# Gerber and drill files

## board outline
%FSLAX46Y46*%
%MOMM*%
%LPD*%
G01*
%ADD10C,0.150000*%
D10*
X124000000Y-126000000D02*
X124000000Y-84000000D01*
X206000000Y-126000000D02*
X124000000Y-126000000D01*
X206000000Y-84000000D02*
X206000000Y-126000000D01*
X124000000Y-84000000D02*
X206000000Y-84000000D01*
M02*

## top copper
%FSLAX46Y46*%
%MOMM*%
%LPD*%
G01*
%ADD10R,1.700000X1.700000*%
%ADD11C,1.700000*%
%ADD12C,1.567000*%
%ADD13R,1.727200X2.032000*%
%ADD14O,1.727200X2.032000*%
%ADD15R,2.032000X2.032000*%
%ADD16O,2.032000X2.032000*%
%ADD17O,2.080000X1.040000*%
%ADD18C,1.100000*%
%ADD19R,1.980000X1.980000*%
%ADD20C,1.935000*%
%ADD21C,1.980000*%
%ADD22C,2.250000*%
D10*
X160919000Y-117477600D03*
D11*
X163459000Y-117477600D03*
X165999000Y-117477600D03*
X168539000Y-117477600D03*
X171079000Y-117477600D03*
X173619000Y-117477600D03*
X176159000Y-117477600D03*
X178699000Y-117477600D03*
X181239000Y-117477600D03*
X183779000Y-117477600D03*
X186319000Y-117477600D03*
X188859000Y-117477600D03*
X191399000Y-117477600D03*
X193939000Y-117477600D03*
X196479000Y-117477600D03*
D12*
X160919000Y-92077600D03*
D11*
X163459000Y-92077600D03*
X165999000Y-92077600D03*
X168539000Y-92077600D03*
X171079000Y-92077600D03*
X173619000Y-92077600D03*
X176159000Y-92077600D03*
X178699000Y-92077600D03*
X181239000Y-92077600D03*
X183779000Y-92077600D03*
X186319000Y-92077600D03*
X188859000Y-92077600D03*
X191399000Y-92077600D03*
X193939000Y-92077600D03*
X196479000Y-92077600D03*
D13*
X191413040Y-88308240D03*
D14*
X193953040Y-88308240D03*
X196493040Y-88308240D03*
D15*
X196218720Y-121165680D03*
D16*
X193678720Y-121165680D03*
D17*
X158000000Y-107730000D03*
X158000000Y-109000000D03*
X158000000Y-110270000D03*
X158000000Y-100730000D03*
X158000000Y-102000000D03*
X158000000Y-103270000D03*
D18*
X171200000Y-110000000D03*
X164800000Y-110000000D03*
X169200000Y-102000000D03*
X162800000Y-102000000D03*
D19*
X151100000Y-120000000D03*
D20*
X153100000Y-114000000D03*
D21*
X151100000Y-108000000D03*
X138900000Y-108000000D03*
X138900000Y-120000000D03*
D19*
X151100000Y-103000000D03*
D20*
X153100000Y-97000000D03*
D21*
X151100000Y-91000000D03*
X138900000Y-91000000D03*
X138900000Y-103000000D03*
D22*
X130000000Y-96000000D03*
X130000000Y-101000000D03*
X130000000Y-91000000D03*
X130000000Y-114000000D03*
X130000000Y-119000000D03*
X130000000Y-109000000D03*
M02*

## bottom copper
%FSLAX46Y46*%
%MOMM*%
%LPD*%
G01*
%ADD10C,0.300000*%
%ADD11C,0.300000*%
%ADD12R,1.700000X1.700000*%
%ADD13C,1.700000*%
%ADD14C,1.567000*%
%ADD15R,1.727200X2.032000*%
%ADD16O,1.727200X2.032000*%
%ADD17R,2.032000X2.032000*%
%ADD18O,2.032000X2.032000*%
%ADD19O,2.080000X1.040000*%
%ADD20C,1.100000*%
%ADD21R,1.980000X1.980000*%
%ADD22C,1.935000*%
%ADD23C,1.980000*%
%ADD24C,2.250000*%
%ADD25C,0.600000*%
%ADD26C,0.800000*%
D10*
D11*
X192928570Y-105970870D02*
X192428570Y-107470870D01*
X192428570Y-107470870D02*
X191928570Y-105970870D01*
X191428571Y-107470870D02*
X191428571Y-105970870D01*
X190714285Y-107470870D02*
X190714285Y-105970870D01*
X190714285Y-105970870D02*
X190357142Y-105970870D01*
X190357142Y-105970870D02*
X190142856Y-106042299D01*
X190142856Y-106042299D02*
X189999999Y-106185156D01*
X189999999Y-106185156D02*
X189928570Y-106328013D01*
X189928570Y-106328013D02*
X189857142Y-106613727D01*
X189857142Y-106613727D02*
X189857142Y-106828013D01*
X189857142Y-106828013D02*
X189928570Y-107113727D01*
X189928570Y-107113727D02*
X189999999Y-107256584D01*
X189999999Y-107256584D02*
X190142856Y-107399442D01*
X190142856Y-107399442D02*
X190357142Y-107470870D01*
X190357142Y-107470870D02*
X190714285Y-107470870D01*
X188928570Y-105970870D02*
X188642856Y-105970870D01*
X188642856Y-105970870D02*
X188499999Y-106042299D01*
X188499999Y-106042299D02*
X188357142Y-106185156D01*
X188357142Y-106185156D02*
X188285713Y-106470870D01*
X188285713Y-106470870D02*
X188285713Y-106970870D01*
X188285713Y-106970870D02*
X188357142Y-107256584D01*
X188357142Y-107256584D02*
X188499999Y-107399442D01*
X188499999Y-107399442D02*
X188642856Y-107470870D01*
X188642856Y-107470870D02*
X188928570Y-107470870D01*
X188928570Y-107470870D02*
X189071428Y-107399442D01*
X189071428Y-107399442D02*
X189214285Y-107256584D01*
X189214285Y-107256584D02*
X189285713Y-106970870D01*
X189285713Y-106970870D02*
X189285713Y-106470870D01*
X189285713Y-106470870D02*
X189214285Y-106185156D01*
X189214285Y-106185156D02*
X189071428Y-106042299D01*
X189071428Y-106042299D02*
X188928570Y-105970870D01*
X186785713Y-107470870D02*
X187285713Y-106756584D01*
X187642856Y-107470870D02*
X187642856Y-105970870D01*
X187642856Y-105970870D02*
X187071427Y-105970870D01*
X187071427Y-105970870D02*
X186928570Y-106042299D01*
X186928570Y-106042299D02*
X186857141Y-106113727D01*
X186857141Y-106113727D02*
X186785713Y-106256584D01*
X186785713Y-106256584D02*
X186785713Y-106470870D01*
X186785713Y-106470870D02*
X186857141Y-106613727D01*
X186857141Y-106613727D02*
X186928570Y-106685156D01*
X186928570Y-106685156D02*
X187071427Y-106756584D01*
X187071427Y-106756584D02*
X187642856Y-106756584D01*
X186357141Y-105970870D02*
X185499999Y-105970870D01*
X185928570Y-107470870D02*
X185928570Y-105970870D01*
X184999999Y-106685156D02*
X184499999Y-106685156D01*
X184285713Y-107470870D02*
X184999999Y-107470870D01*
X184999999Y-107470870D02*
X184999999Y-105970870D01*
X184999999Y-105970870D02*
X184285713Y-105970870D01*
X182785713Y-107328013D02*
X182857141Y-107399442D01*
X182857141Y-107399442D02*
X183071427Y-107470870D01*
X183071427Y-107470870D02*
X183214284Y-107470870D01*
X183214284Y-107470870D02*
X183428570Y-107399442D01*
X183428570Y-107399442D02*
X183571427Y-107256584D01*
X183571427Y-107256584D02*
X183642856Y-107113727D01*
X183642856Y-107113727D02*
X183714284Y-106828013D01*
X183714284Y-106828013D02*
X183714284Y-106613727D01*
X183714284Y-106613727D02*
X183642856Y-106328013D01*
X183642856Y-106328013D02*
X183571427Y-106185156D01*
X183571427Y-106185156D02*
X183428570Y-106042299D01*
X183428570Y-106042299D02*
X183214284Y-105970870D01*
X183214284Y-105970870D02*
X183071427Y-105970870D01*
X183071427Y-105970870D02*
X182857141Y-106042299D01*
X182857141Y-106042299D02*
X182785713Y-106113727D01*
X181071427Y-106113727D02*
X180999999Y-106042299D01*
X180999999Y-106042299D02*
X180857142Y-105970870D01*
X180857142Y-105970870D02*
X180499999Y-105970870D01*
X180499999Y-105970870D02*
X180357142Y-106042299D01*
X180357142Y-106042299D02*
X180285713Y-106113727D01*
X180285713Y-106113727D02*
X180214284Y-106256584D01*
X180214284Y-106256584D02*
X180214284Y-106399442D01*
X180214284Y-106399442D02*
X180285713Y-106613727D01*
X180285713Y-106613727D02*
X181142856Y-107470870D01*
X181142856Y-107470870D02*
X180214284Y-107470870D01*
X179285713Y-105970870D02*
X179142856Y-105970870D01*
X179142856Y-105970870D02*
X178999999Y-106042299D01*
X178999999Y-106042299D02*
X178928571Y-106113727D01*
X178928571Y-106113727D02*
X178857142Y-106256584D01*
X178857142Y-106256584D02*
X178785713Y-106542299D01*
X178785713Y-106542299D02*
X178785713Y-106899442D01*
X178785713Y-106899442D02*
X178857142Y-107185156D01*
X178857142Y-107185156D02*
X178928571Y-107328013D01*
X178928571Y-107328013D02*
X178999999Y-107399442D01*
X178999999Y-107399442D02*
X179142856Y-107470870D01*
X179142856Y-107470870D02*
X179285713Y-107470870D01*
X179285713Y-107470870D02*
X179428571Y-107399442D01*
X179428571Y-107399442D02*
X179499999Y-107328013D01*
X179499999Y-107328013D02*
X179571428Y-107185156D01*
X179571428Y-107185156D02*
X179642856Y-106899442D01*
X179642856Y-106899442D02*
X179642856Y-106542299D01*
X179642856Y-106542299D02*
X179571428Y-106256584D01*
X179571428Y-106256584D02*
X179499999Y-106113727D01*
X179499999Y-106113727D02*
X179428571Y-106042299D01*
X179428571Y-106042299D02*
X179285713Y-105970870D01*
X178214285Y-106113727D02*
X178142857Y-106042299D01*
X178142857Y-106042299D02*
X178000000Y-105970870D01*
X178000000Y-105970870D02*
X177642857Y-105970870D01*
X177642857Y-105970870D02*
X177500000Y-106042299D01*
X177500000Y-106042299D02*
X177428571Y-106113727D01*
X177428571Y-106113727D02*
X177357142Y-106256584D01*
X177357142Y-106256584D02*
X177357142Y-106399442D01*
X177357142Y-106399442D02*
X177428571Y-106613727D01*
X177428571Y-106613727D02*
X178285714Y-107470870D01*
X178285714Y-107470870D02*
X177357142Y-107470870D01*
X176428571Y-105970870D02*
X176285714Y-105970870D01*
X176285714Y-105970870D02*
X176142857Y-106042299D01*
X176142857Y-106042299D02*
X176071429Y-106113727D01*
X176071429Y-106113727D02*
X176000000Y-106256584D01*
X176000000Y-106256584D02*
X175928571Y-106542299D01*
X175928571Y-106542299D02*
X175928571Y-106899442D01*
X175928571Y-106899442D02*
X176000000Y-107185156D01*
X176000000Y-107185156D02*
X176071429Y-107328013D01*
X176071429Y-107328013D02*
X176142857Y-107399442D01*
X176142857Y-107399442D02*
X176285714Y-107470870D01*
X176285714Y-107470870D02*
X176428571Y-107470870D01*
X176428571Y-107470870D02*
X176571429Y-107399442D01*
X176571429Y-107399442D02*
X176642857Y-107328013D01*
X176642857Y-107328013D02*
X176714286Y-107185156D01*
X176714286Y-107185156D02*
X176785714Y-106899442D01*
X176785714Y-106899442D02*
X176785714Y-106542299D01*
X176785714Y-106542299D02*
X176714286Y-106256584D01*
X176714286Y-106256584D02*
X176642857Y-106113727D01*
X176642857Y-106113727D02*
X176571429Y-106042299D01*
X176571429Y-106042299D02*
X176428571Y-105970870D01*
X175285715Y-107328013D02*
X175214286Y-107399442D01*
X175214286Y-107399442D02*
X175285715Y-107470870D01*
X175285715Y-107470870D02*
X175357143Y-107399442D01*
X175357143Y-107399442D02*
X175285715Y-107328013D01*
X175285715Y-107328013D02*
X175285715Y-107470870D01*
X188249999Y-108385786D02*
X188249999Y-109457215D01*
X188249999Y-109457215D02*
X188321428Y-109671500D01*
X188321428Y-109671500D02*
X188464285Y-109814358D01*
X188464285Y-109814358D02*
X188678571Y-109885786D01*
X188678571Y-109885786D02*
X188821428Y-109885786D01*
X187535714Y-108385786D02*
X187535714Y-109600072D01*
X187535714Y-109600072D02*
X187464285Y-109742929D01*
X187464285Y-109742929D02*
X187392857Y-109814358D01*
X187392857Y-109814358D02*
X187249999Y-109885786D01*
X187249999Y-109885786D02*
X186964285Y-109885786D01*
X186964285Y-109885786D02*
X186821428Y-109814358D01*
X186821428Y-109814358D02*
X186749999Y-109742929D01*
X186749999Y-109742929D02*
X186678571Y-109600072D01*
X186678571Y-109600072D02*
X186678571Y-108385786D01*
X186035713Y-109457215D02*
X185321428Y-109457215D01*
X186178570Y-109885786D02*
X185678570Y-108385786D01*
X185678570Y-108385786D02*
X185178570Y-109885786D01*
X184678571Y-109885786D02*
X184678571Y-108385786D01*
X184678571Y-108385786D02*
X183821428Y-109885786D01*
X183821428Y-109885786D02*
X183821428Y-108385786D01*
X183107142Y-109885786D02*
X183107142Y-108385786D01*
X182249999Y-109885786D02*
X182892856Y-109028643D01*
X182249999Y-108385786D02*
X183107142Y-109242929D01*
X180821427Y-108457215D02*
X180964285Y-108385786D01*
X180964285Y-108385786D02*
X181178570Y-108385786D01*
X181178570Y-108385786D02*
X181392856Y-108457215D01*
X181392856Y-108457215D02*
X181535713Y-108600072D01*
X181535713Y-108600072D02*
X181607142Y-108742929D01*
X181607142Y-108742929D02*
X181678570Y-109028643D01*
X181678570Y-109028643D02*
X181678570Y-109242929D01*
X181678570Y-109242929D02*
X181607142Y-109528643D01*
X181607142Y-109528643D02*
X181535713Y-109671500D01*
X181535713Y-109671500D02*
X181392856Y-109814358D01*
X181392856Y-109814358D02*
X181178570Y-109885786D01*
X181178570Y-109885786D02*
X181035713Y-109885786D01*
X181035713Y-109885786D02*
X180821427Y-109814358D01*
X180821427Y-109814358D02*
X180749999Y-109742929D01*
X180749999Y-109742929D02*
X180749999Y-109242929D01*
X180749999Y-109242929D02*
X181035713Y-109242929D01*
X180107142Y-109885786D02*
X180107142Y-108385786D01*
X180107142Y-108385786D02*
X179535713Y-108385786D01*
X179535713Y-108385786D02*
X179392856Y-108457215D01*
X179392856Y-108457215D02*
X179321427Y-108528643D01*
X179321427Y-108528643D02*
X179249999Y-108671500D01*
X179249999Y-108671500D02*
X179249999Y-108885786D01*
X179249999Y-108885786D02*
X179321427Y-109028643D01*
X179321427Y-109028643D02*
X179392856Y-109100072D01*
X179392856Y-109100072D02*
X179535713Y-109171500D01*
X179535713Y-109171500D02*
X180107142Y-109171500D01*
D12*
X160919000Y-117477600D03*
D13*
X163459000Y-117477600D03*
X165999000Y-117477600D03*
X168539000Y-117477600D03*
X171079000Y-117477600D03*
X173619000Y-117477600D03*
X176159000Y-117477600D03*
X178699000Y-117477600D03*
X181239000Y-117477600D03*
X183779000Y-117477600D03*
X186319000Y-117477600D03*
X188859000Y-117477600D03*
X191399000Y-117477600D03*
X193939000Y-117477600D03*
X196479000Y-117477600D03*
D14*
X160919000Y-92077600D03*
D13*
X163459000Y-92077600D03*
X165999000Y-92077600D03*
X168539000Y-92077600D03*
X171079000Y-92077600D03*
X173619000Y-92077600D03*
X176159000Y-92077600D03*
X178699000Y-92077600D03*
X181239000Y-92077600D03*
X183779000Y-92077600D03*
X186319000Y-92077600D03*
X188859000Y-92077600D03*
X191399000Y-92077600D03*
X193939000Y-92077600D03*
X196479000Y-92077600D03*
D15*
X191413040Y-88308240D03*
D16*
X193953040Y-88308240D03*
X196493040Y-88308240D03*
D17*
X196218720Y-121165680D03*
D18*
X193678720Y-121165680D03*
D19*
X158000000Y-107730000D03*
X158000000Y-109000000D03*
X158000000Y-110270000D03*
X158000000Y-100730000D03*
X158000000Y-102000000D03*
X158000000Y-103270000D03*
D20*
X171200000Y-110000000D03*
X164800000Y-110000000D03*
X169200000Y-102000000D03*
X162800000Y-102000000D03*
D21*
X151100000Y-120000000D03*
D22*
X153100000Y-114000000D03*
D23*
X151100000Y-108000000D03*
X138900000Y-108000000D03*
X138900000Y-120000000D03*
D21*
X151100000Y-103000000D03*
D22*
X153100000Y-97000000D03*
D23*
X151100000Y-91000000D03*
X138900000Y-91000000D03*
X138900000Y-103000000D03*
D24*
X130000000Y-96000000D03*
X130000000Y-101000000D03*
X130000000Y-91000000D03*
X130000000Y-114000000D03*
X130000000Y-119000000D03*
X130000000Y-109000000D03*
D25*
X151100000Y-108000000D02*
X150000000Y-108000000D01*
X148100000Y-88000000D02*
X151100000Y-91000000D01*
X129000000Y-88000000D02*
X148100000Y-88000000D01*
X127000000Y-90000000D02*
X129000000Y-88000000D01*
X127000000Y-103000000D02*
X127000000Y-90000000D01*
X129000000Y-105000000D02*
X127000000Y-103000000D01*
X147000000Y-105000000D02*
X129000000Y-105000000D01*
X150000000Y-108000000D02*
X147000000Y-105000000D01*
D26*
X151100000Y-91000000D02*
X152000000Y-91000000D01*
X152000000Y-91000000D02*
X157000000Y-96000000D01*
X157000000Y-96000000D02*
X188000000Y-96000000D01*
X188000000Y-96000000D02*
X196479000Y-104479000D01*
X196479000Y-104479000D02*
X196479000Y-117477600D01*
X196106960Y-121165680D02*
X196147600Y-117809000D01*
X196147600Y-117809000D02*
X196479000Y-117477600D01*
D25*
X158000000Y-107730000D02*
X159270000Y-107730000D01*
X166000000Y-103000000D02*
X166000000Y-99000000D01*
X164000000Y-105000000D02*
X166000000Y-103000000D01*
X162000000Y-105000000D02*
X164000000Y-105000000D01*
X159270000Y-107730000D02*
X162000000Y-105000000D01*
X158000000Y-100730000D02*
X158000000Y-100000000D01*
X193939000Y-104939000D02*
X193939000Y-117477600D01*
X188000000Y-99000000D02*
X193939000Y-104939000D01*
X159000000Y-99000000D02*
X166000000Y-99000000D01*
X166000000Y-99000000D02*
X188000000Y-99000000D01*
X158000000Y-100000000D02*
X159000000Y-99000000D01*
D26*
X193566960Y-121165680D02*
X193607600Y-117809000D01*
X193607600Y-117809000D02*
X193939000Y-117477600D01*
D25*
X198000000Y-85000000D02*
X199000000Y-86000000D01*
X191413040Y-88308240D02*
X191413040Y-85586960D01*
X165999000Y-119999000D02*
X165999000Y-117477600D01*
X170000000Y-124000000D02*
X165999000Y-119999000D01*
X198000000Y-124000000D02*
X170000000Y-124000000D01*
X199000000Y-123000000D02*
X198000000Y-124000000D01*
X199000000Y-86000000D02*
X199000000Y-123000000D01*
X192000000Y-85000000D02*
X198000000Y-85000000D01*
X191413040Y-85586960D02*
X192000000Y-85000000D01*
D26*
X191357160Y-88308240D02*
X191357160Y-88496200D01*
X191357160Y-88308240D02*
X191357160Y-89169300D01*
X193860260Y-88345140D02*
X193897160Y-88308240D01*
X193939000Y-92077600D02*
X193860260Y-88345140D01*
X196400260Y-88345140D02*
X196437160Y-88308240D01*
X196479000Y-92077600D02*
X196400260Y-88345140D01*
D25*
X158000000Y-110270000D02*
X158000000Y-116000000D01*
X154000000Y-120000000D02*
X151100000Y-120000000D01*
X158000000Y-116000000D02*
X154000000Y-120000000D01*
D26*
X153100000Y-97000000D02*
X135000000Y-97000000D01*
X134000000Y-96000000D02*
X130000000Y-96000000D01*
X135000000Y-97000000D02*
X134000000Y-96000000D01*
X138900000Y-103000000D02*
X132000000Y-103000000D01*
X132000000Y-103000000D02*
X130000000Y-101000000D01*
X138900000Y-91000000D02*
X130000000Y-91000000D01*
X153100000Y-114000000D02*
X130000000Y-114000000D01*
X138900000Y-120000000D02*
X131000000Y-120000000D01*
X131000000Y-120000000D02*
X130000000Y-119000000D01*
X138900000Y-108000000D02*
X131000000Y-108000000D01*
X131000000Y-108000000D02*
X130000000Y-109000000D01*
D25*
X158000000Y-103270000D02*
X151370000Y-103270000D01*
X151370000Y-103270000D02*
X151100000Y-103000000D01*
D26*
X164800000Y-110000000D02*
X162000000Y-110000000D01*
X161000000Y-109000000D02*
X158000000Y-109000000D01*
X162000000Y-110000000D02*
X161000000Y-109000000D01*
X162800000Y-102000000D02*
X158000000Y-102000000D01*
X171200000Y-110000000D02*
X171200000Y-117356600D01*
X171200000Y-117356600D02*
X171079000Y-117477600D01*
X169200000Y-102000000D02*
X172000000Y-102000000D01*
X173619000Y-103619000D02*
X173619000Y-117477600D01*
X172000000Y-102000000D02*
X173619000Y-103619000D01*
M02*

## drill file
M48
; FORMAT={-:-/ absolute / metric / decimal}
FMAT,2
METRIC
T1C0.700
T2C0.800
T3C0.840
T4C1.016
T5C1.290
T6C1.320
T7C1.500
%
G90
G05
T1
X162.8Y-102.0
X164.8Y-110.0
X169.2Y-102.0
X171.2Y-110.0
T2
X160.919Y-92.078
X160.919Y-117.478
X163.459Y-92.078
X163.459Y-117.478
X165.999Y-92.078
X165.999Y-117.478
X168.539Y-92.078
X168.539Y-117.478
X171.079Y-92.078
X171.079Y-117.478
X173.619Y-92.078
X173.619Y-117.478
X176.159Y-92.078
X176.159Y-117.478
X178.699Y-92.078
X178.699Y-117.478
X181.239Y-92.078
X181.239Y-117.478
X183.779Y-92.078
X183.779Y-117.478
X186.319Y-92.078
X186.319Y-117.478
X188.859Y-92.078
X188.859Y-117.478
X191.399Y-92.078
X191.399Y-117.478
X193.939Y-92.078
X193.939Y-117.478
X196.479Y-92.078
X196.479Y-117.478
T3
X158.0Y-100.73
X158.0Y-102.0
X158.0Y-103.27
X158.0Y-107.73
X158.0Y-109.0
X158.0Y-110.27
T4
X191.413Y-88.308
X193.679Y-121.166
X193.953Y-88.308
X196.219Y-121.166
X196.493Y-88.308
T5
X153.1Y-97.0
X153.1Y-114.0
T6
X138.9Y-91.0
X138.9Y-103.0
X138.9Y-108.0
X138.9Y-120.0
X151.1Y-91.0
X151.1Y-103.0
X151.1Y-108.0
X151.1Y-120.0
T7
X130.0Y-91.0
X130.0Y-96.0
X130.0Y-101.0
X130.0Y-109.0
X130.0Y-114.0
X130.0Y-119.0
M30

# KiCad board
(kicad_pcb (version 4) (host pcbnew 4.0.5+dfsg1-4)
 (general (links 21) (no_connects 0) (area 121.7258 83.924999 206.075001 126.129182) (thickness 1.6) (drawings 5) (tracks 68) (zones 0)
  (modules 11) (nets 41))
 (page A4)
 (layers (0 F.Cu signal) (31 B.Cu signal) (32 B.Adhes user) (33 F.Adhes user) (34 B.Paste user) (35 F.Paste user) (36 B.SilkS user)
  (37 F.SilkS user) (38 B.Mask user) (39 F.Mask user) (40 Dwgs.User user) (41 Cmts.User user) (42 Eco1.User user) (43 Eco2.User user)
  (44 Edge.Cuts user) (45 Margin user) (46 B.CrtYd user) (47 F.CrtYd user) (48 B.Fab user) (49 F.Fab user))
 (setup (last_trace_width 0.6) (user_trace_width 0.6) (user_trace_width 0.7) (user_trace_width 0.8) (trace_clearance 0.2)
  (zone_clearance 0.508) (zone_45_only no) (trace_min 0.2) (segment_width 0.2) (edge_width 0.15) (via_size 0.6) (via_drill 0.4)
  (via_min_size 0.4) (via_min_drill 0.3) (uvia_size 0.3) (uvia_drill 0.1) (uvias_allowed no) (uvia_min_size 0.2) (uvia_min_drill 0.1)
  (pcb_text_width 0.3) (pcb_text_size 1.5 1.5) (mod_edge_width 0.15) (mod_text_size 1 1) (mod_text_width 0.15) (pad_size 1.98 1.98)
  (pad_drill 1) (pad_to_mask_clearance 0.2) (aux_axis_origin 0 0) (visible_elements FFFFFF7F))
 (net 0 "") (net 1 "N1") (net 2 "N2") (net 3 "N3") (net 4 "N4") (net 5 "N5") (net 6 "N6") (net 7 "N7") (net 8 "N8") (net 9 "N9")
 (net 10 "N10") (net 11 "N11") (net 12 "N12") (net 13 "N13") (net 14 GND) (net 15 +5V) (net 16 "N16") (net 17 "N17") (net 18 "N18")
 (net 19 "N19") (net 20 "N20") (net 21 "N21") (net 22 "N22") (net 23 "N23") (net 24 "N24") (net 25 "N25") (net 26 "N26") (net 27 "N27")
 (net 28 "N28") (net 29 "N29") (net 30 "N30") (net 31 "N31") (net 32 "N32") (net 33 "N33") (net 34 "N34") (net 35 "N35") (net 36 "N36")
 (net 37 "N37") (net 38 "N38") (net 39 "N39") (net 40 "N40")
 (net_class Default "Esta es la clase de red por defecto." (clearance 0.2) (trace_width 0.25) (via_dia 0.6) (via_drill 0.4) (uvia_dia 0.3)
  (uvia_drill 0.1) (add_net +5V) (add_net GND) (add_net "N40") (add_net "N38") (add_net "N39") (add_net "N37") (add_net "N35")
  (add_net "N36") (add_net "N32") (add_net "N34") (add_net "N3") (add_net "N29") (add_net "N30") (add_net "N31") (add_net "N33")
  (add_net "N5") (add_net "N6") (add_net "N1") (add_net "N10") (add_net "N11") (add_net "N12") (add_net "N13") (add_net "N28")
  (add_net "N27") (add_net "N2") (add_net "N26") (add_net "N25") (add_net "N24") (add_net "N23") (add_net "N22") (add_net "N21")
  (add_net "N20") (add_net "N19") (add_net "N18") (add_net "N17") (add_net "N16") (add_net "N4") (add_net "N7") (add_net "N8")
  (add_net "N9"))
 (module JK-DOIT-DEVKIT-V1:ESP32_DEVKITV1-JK (layer F.Cu) (at 180.679 104.7776 90)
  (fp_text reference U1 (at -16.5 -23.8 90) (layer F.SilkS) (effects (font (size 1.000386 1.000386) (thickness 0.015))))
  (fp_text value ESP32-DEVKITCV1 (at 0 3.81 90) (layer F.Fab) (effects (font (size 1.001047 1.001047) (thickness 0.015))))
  (pad 1 thru_hole rect (at -12.7 -19.76 90) (size 1.7 1.7) (drill 0.8) (layers *.Cu *.Mask) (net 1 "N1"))
  (pad 2 thru_hole circle (at -12.7 -17.22 90) (size 1.7 1.7) (drill 0.8) (layers *.Cu *.Mask) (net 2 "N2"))
  (pad 3 thru_hole circle (at -12.7 -14.68 90) (size 1.7 1.7) (drill 0.8) (layers *.Cu *.Mask) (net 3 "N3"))
  (pad 4 thru_hole circle (at -12.7 -12.14 90) (size 1.7 1.7) (drill 0.8) (layers *.Cu *.Mask) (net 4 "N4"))
  (pad 5 thru_hole circle (at -12.7 -9.6 90) (size 1.7 1.7) (drill 0.8) (layers *.Cu *.Mask) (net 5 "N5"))
  (pad 6 thru_hole circle (at -12.7 -7.06 90) (size 1.7 1.7) (drill 0.8) (layers *.Cu *.Mask) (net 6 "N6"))
  (pad 7 thru_hole circle (at -12.7 -4.52 90) (size 1.7 1.7) (drill 0.8) (layers *.Cu *.Mask) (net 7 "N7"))
  (pad 8 thru_hole circle (at -12.7 -1.98 90) (size 1.7 1.7) (drill 0.8) (layers *.Cu *.Mask) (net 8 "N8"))
  (pad 9 thru_hole circle (at -12.7 0.56 90) (size 1.7 1.7) (drill 0.8) (layers *.Cu *.Mask) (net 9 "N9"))
  (pad 10 thru_hole circle (at -12.7 3.1 90) (size 1.7 1.7) (drill 0.8) (layers *.Cu *.Mask) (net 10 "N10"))
  (pad 11 thru_hole circle (at -12.7 5.64 90) (size 1.7 1.7) (drill 0.8) (layers *.Cu *.Mask) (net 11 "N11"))
  (pad 12 thru_hole circle (at -12.7 8.18 90) (size 1.7 1.7) (drill 0.8) (layers *.Cu *.Mask) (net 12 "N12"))
  (pad 13 thru_hole circle (at -12.7 10.72 90) (size 1.7 1.7) (drill 0.8) (layers *.Cu *.Mask) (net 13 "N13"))
  (pad 14 thru_hole circle (at -12.7 13.26 90) (size 1.7 1.7) (drill 0.8) (layers *.Cu *.Mask) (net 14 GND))
  (pad 15 thru_hole circle (at -12.7 15.8 90) (size 1.7 1.7) (drill 0.8) (layers *.Cu *.Mask) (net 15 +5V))
  (pad 30 thru_hole circle (at 12.7 -19.76 90) (size 1.567 1.567) (drill 0.8) (layers *.Cu *.Mask) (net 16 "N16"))
  (pad 29 thru_hole circle (at 12.7 -17.22 90) (size 1.7 1.7) (drill 0.8) (layers *.Cu *.Mask) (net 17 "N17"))
  (pad 28 thru_hole circle (at 12.7 -14.68 90) (size 1.7 1.7) (drill 0.8) (layers *.Cu *.Mask) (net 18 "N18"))
  (pad 27 thru_hole circle (at 12.7 -12.14 90) (size 1.7 1.7) (drill 0.8) (layers *.Cu *.Mask) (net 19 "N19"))
  (pad 26 thru_hole circle (at 12.7 -9.6 90) (size 1.7 1.7) (drill 0.8) (layers *.Cu *.Mask) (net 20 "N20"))
  (pad 25 thru_hole circle (at 12.7 -7.06 90) (size 1.7 1.7) (drill 0.8) (layers *.Cu *.Mask) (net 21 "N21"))
  (pad 24 thru_hole circle (at 12.7 -4.52 90) (size 1.7 1.7) (drill 0.8) (layers *.Cu *.Mask) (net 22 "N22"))
  (pad 23 thru_hole circle (at 12.7 -1.98 90) (size 1.7 1.7) (drill 0.8) (layers *.Cu *.Mask) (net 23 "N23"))
  (pad 22 thru_hole circle (at 12.7 0.56 90) (size 1.7 1.7) (drill 0.8) (layers *.Cu *.Mask) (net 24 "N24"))
  (pad 21 thru_hole circle (at 12.7 3.1 90) (size 1.7 1.7) (drill 0.8) (layers *.Cu *.Mask) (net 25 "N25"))
  (pad 20 thru_hole circle (at 12.7 5.64 90) (size 1.7 1.7) (drill 0.8) (layers *.Cu *.Mask) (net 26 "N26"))
  (pad 19 thru_hole circle (at 12.7 8.18 90) (size 1.7 1.7) (drill 0.8) (layers *.Cu *.Mask) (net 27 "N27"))
  (pad 18 thru_hole circle (at 12.7 10.72 90) (size 1.7 1.7) (drill 0.8) (layers *.Cu *.Mask) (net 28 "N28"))
  (pad 17 thru_hole circle (at 12.7 13.26 90) (size 1.7 1.7) (drill 0.8) (layers *.Cu *.Mask) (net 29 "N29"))
  (pad 16 thru_hole circle (at 12.7 15.8 90) (size 1.7 1.7) (drill 0.8) (layers *.Cu *.Mask) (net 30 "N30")))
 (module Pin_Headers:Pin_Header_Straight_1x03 (layer F.Cu) (at 191.41304 88.30824 90)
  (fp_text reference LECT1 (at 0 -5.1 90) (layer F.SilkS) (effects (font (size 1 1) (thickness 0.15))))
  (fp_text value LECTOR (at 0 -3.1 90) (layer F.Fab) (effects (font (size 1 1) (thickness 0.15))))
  (pad 1 thru_hole rect (at 0 0 90) (size 2.032 1.7272) (drill 1.016) (layers *.Cu *.Mask) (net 3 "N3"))
  (pad 2 thru_hole oval (at 0 2.54 90) (size 2.032 1.7272) (drill 1.016) (layers *.Cu *.Mask) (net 29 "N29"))
  (pad 3 thru_hole oval (at 0 5.08 90) (size 2.032 1.7272) (drill 1.016) (layers *.Cu *.Mask) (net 30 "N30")))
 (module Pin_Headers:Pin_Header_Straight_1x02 (layer F.Cu) (at 196.21872 121.16568 270)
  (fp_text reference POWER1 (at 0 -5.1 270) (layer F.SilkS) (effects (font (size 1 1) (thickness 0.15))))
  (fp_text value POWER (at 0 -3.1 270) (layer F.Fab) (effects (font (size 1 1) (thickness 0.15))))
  (pad 1 thru_hole rect (at 0 0 270) (size 2.032 2.032) (drill 1.016) (layers *.Cu *.Mask) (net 15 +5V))
  (pad 2 thru_hole oval (at 0 2.54 270) (size 2.032 2.032) (drill 1.016) (layers *.Cu *.Mask) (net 14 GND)))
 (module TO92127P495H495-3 (layer F.Cu) (at 158 109 270)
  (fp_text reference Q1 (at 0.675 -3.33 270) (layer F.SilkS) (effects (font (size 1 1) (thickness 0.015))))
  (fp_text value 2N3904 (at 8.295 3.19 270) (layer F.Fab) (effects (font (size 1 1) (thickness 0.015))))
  (pad 1 thru_hole oval (at -1.27 0 270) (size 1.04 2.08) (drill 0.84) (layers *.Cu *.Mask) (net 14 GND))
  (pad 2 thru_hole oval (at 0 0 270) (size 1.04 2.08) (drill 0.84) (layers *.Cu *.Mask) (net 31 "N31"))
  (pad 3 thru_hole oval (at 1.27 0 270) (size 1.04 2.08) (drill 0.84) (layers *.Cu *.Mask) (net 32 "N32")))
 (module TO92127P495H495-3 (layer F.Cu) (at 158 102 270)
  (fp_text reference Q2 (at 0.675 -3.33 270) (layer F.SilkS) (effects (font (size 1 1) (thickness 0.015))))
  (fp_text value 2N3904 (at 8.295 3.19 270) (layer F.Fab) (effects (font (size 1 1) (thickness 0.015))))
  (pad 1 thru_hole oval (at -1.27 0 270) (size 1.04 2.08) (drill 0.84) (layers *.Cu *.Mask) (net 14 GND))
  (pad 2 thru_hole oval (at 0 0 270) (size 1.04 2.08) (drill 0.84) (layers *.Cu *.Mask) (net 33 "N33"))
  (pad 3 thru_hole oval (at 1.27 0 270) (size 1.04 2.08) (drill 0.84) (layers *.Cu *.Mask) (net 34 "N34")))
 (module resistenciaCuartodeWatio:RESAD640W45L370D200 (layer F.Cu) (at 168 110 180)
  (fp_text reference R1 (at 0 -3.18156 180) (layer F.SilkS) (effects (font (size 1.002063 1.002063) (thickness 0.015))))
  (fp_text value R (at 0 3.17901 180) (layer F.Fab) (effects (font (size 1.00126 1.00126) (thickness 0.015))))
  (pad 1 thru_hole circle (at -3.2 0 180) (size 1.1 1.1) (drill 0.7) (layers *.Cu *.Mask) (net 5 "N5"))
  (pad 2 thru_hole circle (at 3.2 0 180) (size 1.1 1.1) (drill 0.7) (layers *.Cu *.Mask) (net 31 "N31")))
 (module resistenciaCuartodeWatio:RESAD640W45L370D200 (layer F.Cu) (at 166 102 180)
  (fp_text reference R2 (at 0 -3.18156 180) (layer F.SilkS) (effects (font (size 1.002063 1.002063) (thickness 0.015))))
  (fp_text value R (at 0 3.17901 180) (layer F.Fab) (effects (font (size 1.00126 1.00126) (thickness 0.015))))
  (pad 1 thru_hole circle (at -3.2 0 180) (size 1.1 1.1) (drill 0.7) (layers *.Cu *.Mask) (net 6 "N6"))
  (pad 2 thru_hole circle (at 3.2 0 180) (size 1.1 1.1) (drill 0.7) (layers *.Cu *.Mask) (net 33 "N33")))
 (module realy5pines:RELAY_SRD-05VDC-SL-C (layer F.Cu) (at 145 114 180)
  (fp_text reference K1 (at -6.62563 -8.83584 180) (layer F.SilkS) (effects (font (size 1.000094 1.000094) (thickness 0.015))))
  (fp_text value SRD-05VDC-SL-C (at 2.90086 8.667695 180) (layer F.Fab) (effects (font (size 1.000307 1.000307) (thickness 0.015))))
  (pad A1 thru_hole rect (at -6.1 -6 180) (size 1.98 1.98) (drill 1.32) (layers *.Cu *.Mask) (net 32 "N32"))
  (pad COM thru_hole circle (at -8.1 0 180) (size 1.935 1.935) (drill 1.29) (layers *.Cu *.Mask) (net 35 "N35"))
  (pad A2 thru_hole circle (at -6.1 6 180) (size 1.98 1.98) (drill 1.32) (layers *.Cu *.Mask) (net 15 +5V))
  (pad NO thru_hole circle (at 6.1 6 180) (size 1.98 1.98) (drill 1.32) (layers *.Cu *.Mask) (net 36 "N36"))
  (pad NC thru_hole circle (at 6.1 -6 180) (size 1.98 1.98) (drill 1.32) (layers *.Cu *.Mask) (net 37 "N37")))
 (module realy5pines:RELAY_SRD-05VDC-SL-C (layer F.Cu) (at 145 97 180)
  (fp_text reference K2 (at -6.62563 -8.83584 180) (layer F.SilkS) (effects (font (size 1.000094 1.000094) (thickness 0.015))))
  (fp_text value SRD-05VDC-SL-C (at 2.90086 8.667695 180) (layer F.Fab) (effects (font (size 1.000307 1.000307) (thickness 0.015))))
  (pad A1 thru_hole rect (at -6.1 -6 180) (size 1.98 1.98) (drill 1.32) (layers *.Cu *.Mask) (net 34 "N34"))
  (pad COM thru_hole circle (at -8.1 0 180) (size 1.935 1.935) (drill 1.29) (layers *.Cu *.Mask) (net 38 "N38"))
  (pad A2 thru_hole circle (at -6.1 6 180) (size 1.98 1.98) (drill 1.32) (layers *.Cu *.Mask) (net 15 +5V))
  (pad NO thru_hole circle (at 6.1 6 180) (size 1.98 1.98) (drill 1.32) (layers *.Cu *.Mask) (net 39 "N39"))
  (pad NC thru_hole circle (at 6.1 -6 180) (size 1.98 1.98) (drill 1.32) (layers *.Cu *.Mask) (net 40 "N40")))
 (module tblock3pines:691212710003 (layer F.Cu) (at 130 96 90)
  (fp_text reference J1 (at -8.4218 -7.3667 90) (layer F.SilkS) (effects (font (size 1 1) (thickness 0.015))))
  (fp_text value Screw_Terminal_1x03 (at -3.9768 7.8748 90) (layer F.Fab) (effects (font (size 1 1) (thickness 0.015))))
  (pad 2 thru_hole circle (at 0 0 90) (size 2.25 2.25) (drill 1.5) (layers *.Cu *.Mask) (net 38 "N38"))
  (pad 1 thru_hole circle (at -5 0 90) (size 2.25 2.25) (drill 1.5) (layers *.Cu *.Mask) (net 40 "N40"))
  (pad 3 thru_hole circle (at 5 0 90) (size 2.25 2.25) (drill 1.5) (layers *.Cu *.Mask) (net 39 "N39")))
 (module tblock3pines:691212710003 (layer F.Cu) (at 130 114 90)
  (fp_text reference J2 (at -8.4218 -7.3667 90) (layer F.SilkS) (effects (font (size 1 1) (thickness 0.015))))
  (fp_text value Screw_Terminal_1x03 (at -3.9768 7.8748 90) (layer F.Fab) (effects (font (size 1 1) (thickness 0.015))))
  (pad 2 thru_hole circle (at 0 0 90) (size 2.25 2.25) (drill 1.5) (layers *.Cu *.Mask) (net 35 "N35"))
  (pad 1 thru_hole circle (at -5 0 90) (size 2.25 2.25) (drill 1.5) (layers *.Cu *.Mask) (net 37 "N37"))
  (pad 3 thru_hole circle (at 5 0 90) (size 2.25 2.25) (drill 1.5) (layers *.Cu *.Mask) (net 36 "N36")))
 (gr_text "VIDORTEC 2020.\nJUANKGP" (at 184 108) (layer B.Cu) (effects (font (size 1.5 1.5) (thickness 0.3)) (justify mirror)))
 (gr_line (start 124 126) (end 124 84) (angle 90) (layer Edge.Cuts) (width 0.15))
 (gr_line (start 206 126) (end 124 126) (angle 90) (layer Edge.Cuts) (width 0.15))
 (gr_line (start 206 84) (end 206 126) (angle 90) (layer Edge.Cuts) (width 0.15))
 (gr_line (start 124 84) (end 206 84) (angle 90) (layer Edge.Cuts) (width 0.15))
 (segment (start 151.1 108) (end 150 108) (width 0.6) (layer B.Cu) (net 15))
 (segment (start 148.1 88) (end 151.1 91) (width 0.6) (layer B.Cu) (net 15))
 (segment (start 129 88) (end 148.1 88) (width 0.6) (layer B.Cu) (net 15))
 (segment (start 127 90) (end 129 88) (width 0.6) (layer B.Cu) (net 15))
 (segment (start 127 103) (end 127 90) (width 0.6) (layer B.Cu) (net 15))
 (segment (start 129 105) (end 127 103) (width 0.6) (layer B.Cu) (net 15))
 (segment (start 147 105) (end 129 105) (width 0.6) (layer B.Cu) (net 15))
 (segment (start 150 108) (end 147 105) (width 0.6) (layer B.Cu) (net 15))
 (segment (start 151.1 91) (end 152 91) (width 0.8) (layer B.Cu) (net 15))
 (segment (start 152 91) (end 157 96) (width 0.8) (layer B.Cu) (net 15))
 (segment (start 157 96) (end 188 96) (width 0.8) (layer B.Cu) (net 15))
 (segment (start 188 96) (end 196.479 104.479) (width 0.8) (layer B.Cu) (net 15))
 (segment (start 196.479 104.479) (end 196.479 117.4776) (width 0.8) (layer B.Cu) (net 15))
 (segment (start 196.10696 121.16568) (end 196.1476 117.809) (width 0.8) (layer B.Cu) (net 15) (status 20))
 (segment (start 196.1476 117.809) (end 196.479 117.4776) (width 0.8) (layer B.Cu) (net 15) (status 30))
 (segment (start 158 107.73) (end 159.27 107.73) (width 0.6) (layer B.Cu) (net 14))
 (segment (start 166 103) (end 166 99) (width 0.6) (layer B.Cu) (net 14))
 (segment (start 164 105) (end 166 103) (width 0.6) (layer B.Cu) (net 14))
 (segment (start 162 105) (end 164 105) (width 0.6) (layer B.Cu) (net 14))
 (segment (start 159.27 107.73) (end 162 105) (width 0.6) (layer B.Cu) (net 14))
 (segment (start 158 100.73) (end 158 100) (width 0.6) (layer B.Cu) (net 14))
 (segment (start 193.939 104.939) (end 193.939 117.4776) (width 0.6) (layer B.Cu) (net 14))
 (segment (start 188 99) (end 193.939 104.939) (width 0.6) (layer B.Cu) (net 14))
 (segment (start 159 99) (end 166 99) (width 0.6) (layer B.Cu) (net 14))
 (segment (start 166 99) (end 188 99) (width 0.6) (layer B.Cu) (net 14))
 (segment (start 158 100) (end 159 99) (width 0.6) (layer B.Cu) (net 14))
 (segment (start 193.56696 121.16568) (end 193.6076 117.809) (width 0.8) (layer B.Cu) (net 14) (status 20))
 (segment (start 193.6076 117.809) (end 193.939 117.4776) (width 0.8) (layer B.Cu) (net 14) (status 30))
 (segment (start 198 85) (end 199 86) (width 0.6) (layer B.Cu) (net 3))
 (segment (start 191.41304 88.30824) (end 191.41304 85.58696) (width 0.6) (layer B.Cu) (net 3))
 (segment (start 165.999 119.999) (end 165.999 117.4776) (width 0.6) (layer B.Cu) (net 3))
 (segment (start 170 124) (end 165.999 119.999) (width 0.6) (layer B.Cu) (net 3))
 (segment (start 198 124) (end 170 124) (width 0.6) (layer B.Cu) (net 3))
 (segment (start 199 123) (end 198 124) (width 0.6) (layer B.Cu) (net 3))
 (segment (start 199 86) (end 199 123) (width 0.6) (layer B.Cu) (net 3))
 (segment (start 192 85) (end 198 85) (width 0.6) (layer B.Cu) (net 3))
 (segment (start 191.41304 85.58696) (end 192 85) (width 0.6) (layer B.Cu) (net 3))
 (segment (start 191.35716 88.30824) (end 191.35716 88.4962) (width 0.8) (layer B.Cu) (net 3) (status 30))
 (segment (start 191.35716 88.30824) (end 191.35716 89.1693) (width 0.8) (layer B.Cu) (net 3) (status 30))
 (segment (start 193.86026 88.34514) (end 193.89716 88.30824) (width 0.8) (layer B.Cu) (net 29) (status 30))
 (segment (start 193.939 92.0776) (end 193.86026 88.34514) (width 0.8) (layer B.Cu) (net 29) (status 10))
 (segment (start 196.40026 88.34514) (end 196.43716 88.30824) (width 0.8) (layer B.Cu) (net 30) (status 30))
 (segment (start 196.479 92.0776) (end 196.40026 88.34514) (width 0.8) (layer B.Cu) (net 30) (status 10))
 (segment (start 158 110.27) (end 158 116) (width 0.6) (layer B.Cu) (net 32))
 (segment (start 154 120) (end 151.1 120) (width 0.6) (layer B.Cu) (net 32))
 (segment (start 158 116) (end 154 120) (width 0.6) (layer B.Cu) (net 32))
 (segment (start 153.1 97) (end 135 97) (width 0.8) (layer B.Cu) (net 38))
 (segment (start 134 96) (end 130 96) (width 0.8) (layer B.Cu) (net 38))
 (segment (start 135 97) (end 134 96) (width 0.8) (layer B.Cu) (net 38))
 (segment (start 138.9 103) (end 132 103) (width 0.8) (layer B.Cu) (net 40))
 (segment (start 132 103) (end 130 101) (width 0.8) (layer B.Cu) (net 40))
 (segment (start 138.9 91) (end 130 91) (width 0.8) (layer B.Cu) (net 39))
 (segment (start 153.1 114) (end 130 114) (width 0.8) (layer B.Cu) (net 35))
 (segment (start 138.9 120) (end 131 120) (width 0.8) (layer B.Cu) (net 37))
 (segment (start 131 120) (end 130 119) (width 0.8) (layer B.Cu) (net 37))
 (segment (start 138.9 108) (end 131 108) (width 0.8) (layer B.Cu) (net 36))
 (segment (start 131 108) (end 130 109) (width 0.8) (layer B.Cu) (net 36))
 (segment (start 158 103.27) (end 151.37 103.27) (width 0.6) (layer B.Cu) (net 34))
 (segment (start 151.37 103.27) (end 151.1 103) (width 0.6) (layer B.Cu) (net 34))
 (segment (start 164.8 110) (end 162 110) (width 0.8) (layer B.Cu) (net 31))
 (segment (start 161 109) (end 158 109) (width 0.8) (layer B.Cu) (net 31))
 (segment (start 162 110) (end 161 109) (width 0.8) (layer B.Cu) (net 31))
 (segment (start 162.8 102) (end 158 102) (width 0.8) (layer B.Cu) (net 33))
 (segment (start 171.2 110) (end 171.2 117.3566) (width 0.8) (layer B.Cu) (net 5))
 (segment (start 171.2 117.3566) (end 171.079 117.4776) (width 0.8) (layer B.Cu) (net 5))
 (segment (start 169.2 102) (end 172 102) (width 0.8) (layer B.Cu) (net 6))
 (segment (start 173.619 103.619) (end 173.619 117.4776) (width 0.8) (layer B.Cu) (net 6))
 (segment (start 172 102) (end 173.619 103.619) (width 0.8) (layer B.Cu) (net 6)))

